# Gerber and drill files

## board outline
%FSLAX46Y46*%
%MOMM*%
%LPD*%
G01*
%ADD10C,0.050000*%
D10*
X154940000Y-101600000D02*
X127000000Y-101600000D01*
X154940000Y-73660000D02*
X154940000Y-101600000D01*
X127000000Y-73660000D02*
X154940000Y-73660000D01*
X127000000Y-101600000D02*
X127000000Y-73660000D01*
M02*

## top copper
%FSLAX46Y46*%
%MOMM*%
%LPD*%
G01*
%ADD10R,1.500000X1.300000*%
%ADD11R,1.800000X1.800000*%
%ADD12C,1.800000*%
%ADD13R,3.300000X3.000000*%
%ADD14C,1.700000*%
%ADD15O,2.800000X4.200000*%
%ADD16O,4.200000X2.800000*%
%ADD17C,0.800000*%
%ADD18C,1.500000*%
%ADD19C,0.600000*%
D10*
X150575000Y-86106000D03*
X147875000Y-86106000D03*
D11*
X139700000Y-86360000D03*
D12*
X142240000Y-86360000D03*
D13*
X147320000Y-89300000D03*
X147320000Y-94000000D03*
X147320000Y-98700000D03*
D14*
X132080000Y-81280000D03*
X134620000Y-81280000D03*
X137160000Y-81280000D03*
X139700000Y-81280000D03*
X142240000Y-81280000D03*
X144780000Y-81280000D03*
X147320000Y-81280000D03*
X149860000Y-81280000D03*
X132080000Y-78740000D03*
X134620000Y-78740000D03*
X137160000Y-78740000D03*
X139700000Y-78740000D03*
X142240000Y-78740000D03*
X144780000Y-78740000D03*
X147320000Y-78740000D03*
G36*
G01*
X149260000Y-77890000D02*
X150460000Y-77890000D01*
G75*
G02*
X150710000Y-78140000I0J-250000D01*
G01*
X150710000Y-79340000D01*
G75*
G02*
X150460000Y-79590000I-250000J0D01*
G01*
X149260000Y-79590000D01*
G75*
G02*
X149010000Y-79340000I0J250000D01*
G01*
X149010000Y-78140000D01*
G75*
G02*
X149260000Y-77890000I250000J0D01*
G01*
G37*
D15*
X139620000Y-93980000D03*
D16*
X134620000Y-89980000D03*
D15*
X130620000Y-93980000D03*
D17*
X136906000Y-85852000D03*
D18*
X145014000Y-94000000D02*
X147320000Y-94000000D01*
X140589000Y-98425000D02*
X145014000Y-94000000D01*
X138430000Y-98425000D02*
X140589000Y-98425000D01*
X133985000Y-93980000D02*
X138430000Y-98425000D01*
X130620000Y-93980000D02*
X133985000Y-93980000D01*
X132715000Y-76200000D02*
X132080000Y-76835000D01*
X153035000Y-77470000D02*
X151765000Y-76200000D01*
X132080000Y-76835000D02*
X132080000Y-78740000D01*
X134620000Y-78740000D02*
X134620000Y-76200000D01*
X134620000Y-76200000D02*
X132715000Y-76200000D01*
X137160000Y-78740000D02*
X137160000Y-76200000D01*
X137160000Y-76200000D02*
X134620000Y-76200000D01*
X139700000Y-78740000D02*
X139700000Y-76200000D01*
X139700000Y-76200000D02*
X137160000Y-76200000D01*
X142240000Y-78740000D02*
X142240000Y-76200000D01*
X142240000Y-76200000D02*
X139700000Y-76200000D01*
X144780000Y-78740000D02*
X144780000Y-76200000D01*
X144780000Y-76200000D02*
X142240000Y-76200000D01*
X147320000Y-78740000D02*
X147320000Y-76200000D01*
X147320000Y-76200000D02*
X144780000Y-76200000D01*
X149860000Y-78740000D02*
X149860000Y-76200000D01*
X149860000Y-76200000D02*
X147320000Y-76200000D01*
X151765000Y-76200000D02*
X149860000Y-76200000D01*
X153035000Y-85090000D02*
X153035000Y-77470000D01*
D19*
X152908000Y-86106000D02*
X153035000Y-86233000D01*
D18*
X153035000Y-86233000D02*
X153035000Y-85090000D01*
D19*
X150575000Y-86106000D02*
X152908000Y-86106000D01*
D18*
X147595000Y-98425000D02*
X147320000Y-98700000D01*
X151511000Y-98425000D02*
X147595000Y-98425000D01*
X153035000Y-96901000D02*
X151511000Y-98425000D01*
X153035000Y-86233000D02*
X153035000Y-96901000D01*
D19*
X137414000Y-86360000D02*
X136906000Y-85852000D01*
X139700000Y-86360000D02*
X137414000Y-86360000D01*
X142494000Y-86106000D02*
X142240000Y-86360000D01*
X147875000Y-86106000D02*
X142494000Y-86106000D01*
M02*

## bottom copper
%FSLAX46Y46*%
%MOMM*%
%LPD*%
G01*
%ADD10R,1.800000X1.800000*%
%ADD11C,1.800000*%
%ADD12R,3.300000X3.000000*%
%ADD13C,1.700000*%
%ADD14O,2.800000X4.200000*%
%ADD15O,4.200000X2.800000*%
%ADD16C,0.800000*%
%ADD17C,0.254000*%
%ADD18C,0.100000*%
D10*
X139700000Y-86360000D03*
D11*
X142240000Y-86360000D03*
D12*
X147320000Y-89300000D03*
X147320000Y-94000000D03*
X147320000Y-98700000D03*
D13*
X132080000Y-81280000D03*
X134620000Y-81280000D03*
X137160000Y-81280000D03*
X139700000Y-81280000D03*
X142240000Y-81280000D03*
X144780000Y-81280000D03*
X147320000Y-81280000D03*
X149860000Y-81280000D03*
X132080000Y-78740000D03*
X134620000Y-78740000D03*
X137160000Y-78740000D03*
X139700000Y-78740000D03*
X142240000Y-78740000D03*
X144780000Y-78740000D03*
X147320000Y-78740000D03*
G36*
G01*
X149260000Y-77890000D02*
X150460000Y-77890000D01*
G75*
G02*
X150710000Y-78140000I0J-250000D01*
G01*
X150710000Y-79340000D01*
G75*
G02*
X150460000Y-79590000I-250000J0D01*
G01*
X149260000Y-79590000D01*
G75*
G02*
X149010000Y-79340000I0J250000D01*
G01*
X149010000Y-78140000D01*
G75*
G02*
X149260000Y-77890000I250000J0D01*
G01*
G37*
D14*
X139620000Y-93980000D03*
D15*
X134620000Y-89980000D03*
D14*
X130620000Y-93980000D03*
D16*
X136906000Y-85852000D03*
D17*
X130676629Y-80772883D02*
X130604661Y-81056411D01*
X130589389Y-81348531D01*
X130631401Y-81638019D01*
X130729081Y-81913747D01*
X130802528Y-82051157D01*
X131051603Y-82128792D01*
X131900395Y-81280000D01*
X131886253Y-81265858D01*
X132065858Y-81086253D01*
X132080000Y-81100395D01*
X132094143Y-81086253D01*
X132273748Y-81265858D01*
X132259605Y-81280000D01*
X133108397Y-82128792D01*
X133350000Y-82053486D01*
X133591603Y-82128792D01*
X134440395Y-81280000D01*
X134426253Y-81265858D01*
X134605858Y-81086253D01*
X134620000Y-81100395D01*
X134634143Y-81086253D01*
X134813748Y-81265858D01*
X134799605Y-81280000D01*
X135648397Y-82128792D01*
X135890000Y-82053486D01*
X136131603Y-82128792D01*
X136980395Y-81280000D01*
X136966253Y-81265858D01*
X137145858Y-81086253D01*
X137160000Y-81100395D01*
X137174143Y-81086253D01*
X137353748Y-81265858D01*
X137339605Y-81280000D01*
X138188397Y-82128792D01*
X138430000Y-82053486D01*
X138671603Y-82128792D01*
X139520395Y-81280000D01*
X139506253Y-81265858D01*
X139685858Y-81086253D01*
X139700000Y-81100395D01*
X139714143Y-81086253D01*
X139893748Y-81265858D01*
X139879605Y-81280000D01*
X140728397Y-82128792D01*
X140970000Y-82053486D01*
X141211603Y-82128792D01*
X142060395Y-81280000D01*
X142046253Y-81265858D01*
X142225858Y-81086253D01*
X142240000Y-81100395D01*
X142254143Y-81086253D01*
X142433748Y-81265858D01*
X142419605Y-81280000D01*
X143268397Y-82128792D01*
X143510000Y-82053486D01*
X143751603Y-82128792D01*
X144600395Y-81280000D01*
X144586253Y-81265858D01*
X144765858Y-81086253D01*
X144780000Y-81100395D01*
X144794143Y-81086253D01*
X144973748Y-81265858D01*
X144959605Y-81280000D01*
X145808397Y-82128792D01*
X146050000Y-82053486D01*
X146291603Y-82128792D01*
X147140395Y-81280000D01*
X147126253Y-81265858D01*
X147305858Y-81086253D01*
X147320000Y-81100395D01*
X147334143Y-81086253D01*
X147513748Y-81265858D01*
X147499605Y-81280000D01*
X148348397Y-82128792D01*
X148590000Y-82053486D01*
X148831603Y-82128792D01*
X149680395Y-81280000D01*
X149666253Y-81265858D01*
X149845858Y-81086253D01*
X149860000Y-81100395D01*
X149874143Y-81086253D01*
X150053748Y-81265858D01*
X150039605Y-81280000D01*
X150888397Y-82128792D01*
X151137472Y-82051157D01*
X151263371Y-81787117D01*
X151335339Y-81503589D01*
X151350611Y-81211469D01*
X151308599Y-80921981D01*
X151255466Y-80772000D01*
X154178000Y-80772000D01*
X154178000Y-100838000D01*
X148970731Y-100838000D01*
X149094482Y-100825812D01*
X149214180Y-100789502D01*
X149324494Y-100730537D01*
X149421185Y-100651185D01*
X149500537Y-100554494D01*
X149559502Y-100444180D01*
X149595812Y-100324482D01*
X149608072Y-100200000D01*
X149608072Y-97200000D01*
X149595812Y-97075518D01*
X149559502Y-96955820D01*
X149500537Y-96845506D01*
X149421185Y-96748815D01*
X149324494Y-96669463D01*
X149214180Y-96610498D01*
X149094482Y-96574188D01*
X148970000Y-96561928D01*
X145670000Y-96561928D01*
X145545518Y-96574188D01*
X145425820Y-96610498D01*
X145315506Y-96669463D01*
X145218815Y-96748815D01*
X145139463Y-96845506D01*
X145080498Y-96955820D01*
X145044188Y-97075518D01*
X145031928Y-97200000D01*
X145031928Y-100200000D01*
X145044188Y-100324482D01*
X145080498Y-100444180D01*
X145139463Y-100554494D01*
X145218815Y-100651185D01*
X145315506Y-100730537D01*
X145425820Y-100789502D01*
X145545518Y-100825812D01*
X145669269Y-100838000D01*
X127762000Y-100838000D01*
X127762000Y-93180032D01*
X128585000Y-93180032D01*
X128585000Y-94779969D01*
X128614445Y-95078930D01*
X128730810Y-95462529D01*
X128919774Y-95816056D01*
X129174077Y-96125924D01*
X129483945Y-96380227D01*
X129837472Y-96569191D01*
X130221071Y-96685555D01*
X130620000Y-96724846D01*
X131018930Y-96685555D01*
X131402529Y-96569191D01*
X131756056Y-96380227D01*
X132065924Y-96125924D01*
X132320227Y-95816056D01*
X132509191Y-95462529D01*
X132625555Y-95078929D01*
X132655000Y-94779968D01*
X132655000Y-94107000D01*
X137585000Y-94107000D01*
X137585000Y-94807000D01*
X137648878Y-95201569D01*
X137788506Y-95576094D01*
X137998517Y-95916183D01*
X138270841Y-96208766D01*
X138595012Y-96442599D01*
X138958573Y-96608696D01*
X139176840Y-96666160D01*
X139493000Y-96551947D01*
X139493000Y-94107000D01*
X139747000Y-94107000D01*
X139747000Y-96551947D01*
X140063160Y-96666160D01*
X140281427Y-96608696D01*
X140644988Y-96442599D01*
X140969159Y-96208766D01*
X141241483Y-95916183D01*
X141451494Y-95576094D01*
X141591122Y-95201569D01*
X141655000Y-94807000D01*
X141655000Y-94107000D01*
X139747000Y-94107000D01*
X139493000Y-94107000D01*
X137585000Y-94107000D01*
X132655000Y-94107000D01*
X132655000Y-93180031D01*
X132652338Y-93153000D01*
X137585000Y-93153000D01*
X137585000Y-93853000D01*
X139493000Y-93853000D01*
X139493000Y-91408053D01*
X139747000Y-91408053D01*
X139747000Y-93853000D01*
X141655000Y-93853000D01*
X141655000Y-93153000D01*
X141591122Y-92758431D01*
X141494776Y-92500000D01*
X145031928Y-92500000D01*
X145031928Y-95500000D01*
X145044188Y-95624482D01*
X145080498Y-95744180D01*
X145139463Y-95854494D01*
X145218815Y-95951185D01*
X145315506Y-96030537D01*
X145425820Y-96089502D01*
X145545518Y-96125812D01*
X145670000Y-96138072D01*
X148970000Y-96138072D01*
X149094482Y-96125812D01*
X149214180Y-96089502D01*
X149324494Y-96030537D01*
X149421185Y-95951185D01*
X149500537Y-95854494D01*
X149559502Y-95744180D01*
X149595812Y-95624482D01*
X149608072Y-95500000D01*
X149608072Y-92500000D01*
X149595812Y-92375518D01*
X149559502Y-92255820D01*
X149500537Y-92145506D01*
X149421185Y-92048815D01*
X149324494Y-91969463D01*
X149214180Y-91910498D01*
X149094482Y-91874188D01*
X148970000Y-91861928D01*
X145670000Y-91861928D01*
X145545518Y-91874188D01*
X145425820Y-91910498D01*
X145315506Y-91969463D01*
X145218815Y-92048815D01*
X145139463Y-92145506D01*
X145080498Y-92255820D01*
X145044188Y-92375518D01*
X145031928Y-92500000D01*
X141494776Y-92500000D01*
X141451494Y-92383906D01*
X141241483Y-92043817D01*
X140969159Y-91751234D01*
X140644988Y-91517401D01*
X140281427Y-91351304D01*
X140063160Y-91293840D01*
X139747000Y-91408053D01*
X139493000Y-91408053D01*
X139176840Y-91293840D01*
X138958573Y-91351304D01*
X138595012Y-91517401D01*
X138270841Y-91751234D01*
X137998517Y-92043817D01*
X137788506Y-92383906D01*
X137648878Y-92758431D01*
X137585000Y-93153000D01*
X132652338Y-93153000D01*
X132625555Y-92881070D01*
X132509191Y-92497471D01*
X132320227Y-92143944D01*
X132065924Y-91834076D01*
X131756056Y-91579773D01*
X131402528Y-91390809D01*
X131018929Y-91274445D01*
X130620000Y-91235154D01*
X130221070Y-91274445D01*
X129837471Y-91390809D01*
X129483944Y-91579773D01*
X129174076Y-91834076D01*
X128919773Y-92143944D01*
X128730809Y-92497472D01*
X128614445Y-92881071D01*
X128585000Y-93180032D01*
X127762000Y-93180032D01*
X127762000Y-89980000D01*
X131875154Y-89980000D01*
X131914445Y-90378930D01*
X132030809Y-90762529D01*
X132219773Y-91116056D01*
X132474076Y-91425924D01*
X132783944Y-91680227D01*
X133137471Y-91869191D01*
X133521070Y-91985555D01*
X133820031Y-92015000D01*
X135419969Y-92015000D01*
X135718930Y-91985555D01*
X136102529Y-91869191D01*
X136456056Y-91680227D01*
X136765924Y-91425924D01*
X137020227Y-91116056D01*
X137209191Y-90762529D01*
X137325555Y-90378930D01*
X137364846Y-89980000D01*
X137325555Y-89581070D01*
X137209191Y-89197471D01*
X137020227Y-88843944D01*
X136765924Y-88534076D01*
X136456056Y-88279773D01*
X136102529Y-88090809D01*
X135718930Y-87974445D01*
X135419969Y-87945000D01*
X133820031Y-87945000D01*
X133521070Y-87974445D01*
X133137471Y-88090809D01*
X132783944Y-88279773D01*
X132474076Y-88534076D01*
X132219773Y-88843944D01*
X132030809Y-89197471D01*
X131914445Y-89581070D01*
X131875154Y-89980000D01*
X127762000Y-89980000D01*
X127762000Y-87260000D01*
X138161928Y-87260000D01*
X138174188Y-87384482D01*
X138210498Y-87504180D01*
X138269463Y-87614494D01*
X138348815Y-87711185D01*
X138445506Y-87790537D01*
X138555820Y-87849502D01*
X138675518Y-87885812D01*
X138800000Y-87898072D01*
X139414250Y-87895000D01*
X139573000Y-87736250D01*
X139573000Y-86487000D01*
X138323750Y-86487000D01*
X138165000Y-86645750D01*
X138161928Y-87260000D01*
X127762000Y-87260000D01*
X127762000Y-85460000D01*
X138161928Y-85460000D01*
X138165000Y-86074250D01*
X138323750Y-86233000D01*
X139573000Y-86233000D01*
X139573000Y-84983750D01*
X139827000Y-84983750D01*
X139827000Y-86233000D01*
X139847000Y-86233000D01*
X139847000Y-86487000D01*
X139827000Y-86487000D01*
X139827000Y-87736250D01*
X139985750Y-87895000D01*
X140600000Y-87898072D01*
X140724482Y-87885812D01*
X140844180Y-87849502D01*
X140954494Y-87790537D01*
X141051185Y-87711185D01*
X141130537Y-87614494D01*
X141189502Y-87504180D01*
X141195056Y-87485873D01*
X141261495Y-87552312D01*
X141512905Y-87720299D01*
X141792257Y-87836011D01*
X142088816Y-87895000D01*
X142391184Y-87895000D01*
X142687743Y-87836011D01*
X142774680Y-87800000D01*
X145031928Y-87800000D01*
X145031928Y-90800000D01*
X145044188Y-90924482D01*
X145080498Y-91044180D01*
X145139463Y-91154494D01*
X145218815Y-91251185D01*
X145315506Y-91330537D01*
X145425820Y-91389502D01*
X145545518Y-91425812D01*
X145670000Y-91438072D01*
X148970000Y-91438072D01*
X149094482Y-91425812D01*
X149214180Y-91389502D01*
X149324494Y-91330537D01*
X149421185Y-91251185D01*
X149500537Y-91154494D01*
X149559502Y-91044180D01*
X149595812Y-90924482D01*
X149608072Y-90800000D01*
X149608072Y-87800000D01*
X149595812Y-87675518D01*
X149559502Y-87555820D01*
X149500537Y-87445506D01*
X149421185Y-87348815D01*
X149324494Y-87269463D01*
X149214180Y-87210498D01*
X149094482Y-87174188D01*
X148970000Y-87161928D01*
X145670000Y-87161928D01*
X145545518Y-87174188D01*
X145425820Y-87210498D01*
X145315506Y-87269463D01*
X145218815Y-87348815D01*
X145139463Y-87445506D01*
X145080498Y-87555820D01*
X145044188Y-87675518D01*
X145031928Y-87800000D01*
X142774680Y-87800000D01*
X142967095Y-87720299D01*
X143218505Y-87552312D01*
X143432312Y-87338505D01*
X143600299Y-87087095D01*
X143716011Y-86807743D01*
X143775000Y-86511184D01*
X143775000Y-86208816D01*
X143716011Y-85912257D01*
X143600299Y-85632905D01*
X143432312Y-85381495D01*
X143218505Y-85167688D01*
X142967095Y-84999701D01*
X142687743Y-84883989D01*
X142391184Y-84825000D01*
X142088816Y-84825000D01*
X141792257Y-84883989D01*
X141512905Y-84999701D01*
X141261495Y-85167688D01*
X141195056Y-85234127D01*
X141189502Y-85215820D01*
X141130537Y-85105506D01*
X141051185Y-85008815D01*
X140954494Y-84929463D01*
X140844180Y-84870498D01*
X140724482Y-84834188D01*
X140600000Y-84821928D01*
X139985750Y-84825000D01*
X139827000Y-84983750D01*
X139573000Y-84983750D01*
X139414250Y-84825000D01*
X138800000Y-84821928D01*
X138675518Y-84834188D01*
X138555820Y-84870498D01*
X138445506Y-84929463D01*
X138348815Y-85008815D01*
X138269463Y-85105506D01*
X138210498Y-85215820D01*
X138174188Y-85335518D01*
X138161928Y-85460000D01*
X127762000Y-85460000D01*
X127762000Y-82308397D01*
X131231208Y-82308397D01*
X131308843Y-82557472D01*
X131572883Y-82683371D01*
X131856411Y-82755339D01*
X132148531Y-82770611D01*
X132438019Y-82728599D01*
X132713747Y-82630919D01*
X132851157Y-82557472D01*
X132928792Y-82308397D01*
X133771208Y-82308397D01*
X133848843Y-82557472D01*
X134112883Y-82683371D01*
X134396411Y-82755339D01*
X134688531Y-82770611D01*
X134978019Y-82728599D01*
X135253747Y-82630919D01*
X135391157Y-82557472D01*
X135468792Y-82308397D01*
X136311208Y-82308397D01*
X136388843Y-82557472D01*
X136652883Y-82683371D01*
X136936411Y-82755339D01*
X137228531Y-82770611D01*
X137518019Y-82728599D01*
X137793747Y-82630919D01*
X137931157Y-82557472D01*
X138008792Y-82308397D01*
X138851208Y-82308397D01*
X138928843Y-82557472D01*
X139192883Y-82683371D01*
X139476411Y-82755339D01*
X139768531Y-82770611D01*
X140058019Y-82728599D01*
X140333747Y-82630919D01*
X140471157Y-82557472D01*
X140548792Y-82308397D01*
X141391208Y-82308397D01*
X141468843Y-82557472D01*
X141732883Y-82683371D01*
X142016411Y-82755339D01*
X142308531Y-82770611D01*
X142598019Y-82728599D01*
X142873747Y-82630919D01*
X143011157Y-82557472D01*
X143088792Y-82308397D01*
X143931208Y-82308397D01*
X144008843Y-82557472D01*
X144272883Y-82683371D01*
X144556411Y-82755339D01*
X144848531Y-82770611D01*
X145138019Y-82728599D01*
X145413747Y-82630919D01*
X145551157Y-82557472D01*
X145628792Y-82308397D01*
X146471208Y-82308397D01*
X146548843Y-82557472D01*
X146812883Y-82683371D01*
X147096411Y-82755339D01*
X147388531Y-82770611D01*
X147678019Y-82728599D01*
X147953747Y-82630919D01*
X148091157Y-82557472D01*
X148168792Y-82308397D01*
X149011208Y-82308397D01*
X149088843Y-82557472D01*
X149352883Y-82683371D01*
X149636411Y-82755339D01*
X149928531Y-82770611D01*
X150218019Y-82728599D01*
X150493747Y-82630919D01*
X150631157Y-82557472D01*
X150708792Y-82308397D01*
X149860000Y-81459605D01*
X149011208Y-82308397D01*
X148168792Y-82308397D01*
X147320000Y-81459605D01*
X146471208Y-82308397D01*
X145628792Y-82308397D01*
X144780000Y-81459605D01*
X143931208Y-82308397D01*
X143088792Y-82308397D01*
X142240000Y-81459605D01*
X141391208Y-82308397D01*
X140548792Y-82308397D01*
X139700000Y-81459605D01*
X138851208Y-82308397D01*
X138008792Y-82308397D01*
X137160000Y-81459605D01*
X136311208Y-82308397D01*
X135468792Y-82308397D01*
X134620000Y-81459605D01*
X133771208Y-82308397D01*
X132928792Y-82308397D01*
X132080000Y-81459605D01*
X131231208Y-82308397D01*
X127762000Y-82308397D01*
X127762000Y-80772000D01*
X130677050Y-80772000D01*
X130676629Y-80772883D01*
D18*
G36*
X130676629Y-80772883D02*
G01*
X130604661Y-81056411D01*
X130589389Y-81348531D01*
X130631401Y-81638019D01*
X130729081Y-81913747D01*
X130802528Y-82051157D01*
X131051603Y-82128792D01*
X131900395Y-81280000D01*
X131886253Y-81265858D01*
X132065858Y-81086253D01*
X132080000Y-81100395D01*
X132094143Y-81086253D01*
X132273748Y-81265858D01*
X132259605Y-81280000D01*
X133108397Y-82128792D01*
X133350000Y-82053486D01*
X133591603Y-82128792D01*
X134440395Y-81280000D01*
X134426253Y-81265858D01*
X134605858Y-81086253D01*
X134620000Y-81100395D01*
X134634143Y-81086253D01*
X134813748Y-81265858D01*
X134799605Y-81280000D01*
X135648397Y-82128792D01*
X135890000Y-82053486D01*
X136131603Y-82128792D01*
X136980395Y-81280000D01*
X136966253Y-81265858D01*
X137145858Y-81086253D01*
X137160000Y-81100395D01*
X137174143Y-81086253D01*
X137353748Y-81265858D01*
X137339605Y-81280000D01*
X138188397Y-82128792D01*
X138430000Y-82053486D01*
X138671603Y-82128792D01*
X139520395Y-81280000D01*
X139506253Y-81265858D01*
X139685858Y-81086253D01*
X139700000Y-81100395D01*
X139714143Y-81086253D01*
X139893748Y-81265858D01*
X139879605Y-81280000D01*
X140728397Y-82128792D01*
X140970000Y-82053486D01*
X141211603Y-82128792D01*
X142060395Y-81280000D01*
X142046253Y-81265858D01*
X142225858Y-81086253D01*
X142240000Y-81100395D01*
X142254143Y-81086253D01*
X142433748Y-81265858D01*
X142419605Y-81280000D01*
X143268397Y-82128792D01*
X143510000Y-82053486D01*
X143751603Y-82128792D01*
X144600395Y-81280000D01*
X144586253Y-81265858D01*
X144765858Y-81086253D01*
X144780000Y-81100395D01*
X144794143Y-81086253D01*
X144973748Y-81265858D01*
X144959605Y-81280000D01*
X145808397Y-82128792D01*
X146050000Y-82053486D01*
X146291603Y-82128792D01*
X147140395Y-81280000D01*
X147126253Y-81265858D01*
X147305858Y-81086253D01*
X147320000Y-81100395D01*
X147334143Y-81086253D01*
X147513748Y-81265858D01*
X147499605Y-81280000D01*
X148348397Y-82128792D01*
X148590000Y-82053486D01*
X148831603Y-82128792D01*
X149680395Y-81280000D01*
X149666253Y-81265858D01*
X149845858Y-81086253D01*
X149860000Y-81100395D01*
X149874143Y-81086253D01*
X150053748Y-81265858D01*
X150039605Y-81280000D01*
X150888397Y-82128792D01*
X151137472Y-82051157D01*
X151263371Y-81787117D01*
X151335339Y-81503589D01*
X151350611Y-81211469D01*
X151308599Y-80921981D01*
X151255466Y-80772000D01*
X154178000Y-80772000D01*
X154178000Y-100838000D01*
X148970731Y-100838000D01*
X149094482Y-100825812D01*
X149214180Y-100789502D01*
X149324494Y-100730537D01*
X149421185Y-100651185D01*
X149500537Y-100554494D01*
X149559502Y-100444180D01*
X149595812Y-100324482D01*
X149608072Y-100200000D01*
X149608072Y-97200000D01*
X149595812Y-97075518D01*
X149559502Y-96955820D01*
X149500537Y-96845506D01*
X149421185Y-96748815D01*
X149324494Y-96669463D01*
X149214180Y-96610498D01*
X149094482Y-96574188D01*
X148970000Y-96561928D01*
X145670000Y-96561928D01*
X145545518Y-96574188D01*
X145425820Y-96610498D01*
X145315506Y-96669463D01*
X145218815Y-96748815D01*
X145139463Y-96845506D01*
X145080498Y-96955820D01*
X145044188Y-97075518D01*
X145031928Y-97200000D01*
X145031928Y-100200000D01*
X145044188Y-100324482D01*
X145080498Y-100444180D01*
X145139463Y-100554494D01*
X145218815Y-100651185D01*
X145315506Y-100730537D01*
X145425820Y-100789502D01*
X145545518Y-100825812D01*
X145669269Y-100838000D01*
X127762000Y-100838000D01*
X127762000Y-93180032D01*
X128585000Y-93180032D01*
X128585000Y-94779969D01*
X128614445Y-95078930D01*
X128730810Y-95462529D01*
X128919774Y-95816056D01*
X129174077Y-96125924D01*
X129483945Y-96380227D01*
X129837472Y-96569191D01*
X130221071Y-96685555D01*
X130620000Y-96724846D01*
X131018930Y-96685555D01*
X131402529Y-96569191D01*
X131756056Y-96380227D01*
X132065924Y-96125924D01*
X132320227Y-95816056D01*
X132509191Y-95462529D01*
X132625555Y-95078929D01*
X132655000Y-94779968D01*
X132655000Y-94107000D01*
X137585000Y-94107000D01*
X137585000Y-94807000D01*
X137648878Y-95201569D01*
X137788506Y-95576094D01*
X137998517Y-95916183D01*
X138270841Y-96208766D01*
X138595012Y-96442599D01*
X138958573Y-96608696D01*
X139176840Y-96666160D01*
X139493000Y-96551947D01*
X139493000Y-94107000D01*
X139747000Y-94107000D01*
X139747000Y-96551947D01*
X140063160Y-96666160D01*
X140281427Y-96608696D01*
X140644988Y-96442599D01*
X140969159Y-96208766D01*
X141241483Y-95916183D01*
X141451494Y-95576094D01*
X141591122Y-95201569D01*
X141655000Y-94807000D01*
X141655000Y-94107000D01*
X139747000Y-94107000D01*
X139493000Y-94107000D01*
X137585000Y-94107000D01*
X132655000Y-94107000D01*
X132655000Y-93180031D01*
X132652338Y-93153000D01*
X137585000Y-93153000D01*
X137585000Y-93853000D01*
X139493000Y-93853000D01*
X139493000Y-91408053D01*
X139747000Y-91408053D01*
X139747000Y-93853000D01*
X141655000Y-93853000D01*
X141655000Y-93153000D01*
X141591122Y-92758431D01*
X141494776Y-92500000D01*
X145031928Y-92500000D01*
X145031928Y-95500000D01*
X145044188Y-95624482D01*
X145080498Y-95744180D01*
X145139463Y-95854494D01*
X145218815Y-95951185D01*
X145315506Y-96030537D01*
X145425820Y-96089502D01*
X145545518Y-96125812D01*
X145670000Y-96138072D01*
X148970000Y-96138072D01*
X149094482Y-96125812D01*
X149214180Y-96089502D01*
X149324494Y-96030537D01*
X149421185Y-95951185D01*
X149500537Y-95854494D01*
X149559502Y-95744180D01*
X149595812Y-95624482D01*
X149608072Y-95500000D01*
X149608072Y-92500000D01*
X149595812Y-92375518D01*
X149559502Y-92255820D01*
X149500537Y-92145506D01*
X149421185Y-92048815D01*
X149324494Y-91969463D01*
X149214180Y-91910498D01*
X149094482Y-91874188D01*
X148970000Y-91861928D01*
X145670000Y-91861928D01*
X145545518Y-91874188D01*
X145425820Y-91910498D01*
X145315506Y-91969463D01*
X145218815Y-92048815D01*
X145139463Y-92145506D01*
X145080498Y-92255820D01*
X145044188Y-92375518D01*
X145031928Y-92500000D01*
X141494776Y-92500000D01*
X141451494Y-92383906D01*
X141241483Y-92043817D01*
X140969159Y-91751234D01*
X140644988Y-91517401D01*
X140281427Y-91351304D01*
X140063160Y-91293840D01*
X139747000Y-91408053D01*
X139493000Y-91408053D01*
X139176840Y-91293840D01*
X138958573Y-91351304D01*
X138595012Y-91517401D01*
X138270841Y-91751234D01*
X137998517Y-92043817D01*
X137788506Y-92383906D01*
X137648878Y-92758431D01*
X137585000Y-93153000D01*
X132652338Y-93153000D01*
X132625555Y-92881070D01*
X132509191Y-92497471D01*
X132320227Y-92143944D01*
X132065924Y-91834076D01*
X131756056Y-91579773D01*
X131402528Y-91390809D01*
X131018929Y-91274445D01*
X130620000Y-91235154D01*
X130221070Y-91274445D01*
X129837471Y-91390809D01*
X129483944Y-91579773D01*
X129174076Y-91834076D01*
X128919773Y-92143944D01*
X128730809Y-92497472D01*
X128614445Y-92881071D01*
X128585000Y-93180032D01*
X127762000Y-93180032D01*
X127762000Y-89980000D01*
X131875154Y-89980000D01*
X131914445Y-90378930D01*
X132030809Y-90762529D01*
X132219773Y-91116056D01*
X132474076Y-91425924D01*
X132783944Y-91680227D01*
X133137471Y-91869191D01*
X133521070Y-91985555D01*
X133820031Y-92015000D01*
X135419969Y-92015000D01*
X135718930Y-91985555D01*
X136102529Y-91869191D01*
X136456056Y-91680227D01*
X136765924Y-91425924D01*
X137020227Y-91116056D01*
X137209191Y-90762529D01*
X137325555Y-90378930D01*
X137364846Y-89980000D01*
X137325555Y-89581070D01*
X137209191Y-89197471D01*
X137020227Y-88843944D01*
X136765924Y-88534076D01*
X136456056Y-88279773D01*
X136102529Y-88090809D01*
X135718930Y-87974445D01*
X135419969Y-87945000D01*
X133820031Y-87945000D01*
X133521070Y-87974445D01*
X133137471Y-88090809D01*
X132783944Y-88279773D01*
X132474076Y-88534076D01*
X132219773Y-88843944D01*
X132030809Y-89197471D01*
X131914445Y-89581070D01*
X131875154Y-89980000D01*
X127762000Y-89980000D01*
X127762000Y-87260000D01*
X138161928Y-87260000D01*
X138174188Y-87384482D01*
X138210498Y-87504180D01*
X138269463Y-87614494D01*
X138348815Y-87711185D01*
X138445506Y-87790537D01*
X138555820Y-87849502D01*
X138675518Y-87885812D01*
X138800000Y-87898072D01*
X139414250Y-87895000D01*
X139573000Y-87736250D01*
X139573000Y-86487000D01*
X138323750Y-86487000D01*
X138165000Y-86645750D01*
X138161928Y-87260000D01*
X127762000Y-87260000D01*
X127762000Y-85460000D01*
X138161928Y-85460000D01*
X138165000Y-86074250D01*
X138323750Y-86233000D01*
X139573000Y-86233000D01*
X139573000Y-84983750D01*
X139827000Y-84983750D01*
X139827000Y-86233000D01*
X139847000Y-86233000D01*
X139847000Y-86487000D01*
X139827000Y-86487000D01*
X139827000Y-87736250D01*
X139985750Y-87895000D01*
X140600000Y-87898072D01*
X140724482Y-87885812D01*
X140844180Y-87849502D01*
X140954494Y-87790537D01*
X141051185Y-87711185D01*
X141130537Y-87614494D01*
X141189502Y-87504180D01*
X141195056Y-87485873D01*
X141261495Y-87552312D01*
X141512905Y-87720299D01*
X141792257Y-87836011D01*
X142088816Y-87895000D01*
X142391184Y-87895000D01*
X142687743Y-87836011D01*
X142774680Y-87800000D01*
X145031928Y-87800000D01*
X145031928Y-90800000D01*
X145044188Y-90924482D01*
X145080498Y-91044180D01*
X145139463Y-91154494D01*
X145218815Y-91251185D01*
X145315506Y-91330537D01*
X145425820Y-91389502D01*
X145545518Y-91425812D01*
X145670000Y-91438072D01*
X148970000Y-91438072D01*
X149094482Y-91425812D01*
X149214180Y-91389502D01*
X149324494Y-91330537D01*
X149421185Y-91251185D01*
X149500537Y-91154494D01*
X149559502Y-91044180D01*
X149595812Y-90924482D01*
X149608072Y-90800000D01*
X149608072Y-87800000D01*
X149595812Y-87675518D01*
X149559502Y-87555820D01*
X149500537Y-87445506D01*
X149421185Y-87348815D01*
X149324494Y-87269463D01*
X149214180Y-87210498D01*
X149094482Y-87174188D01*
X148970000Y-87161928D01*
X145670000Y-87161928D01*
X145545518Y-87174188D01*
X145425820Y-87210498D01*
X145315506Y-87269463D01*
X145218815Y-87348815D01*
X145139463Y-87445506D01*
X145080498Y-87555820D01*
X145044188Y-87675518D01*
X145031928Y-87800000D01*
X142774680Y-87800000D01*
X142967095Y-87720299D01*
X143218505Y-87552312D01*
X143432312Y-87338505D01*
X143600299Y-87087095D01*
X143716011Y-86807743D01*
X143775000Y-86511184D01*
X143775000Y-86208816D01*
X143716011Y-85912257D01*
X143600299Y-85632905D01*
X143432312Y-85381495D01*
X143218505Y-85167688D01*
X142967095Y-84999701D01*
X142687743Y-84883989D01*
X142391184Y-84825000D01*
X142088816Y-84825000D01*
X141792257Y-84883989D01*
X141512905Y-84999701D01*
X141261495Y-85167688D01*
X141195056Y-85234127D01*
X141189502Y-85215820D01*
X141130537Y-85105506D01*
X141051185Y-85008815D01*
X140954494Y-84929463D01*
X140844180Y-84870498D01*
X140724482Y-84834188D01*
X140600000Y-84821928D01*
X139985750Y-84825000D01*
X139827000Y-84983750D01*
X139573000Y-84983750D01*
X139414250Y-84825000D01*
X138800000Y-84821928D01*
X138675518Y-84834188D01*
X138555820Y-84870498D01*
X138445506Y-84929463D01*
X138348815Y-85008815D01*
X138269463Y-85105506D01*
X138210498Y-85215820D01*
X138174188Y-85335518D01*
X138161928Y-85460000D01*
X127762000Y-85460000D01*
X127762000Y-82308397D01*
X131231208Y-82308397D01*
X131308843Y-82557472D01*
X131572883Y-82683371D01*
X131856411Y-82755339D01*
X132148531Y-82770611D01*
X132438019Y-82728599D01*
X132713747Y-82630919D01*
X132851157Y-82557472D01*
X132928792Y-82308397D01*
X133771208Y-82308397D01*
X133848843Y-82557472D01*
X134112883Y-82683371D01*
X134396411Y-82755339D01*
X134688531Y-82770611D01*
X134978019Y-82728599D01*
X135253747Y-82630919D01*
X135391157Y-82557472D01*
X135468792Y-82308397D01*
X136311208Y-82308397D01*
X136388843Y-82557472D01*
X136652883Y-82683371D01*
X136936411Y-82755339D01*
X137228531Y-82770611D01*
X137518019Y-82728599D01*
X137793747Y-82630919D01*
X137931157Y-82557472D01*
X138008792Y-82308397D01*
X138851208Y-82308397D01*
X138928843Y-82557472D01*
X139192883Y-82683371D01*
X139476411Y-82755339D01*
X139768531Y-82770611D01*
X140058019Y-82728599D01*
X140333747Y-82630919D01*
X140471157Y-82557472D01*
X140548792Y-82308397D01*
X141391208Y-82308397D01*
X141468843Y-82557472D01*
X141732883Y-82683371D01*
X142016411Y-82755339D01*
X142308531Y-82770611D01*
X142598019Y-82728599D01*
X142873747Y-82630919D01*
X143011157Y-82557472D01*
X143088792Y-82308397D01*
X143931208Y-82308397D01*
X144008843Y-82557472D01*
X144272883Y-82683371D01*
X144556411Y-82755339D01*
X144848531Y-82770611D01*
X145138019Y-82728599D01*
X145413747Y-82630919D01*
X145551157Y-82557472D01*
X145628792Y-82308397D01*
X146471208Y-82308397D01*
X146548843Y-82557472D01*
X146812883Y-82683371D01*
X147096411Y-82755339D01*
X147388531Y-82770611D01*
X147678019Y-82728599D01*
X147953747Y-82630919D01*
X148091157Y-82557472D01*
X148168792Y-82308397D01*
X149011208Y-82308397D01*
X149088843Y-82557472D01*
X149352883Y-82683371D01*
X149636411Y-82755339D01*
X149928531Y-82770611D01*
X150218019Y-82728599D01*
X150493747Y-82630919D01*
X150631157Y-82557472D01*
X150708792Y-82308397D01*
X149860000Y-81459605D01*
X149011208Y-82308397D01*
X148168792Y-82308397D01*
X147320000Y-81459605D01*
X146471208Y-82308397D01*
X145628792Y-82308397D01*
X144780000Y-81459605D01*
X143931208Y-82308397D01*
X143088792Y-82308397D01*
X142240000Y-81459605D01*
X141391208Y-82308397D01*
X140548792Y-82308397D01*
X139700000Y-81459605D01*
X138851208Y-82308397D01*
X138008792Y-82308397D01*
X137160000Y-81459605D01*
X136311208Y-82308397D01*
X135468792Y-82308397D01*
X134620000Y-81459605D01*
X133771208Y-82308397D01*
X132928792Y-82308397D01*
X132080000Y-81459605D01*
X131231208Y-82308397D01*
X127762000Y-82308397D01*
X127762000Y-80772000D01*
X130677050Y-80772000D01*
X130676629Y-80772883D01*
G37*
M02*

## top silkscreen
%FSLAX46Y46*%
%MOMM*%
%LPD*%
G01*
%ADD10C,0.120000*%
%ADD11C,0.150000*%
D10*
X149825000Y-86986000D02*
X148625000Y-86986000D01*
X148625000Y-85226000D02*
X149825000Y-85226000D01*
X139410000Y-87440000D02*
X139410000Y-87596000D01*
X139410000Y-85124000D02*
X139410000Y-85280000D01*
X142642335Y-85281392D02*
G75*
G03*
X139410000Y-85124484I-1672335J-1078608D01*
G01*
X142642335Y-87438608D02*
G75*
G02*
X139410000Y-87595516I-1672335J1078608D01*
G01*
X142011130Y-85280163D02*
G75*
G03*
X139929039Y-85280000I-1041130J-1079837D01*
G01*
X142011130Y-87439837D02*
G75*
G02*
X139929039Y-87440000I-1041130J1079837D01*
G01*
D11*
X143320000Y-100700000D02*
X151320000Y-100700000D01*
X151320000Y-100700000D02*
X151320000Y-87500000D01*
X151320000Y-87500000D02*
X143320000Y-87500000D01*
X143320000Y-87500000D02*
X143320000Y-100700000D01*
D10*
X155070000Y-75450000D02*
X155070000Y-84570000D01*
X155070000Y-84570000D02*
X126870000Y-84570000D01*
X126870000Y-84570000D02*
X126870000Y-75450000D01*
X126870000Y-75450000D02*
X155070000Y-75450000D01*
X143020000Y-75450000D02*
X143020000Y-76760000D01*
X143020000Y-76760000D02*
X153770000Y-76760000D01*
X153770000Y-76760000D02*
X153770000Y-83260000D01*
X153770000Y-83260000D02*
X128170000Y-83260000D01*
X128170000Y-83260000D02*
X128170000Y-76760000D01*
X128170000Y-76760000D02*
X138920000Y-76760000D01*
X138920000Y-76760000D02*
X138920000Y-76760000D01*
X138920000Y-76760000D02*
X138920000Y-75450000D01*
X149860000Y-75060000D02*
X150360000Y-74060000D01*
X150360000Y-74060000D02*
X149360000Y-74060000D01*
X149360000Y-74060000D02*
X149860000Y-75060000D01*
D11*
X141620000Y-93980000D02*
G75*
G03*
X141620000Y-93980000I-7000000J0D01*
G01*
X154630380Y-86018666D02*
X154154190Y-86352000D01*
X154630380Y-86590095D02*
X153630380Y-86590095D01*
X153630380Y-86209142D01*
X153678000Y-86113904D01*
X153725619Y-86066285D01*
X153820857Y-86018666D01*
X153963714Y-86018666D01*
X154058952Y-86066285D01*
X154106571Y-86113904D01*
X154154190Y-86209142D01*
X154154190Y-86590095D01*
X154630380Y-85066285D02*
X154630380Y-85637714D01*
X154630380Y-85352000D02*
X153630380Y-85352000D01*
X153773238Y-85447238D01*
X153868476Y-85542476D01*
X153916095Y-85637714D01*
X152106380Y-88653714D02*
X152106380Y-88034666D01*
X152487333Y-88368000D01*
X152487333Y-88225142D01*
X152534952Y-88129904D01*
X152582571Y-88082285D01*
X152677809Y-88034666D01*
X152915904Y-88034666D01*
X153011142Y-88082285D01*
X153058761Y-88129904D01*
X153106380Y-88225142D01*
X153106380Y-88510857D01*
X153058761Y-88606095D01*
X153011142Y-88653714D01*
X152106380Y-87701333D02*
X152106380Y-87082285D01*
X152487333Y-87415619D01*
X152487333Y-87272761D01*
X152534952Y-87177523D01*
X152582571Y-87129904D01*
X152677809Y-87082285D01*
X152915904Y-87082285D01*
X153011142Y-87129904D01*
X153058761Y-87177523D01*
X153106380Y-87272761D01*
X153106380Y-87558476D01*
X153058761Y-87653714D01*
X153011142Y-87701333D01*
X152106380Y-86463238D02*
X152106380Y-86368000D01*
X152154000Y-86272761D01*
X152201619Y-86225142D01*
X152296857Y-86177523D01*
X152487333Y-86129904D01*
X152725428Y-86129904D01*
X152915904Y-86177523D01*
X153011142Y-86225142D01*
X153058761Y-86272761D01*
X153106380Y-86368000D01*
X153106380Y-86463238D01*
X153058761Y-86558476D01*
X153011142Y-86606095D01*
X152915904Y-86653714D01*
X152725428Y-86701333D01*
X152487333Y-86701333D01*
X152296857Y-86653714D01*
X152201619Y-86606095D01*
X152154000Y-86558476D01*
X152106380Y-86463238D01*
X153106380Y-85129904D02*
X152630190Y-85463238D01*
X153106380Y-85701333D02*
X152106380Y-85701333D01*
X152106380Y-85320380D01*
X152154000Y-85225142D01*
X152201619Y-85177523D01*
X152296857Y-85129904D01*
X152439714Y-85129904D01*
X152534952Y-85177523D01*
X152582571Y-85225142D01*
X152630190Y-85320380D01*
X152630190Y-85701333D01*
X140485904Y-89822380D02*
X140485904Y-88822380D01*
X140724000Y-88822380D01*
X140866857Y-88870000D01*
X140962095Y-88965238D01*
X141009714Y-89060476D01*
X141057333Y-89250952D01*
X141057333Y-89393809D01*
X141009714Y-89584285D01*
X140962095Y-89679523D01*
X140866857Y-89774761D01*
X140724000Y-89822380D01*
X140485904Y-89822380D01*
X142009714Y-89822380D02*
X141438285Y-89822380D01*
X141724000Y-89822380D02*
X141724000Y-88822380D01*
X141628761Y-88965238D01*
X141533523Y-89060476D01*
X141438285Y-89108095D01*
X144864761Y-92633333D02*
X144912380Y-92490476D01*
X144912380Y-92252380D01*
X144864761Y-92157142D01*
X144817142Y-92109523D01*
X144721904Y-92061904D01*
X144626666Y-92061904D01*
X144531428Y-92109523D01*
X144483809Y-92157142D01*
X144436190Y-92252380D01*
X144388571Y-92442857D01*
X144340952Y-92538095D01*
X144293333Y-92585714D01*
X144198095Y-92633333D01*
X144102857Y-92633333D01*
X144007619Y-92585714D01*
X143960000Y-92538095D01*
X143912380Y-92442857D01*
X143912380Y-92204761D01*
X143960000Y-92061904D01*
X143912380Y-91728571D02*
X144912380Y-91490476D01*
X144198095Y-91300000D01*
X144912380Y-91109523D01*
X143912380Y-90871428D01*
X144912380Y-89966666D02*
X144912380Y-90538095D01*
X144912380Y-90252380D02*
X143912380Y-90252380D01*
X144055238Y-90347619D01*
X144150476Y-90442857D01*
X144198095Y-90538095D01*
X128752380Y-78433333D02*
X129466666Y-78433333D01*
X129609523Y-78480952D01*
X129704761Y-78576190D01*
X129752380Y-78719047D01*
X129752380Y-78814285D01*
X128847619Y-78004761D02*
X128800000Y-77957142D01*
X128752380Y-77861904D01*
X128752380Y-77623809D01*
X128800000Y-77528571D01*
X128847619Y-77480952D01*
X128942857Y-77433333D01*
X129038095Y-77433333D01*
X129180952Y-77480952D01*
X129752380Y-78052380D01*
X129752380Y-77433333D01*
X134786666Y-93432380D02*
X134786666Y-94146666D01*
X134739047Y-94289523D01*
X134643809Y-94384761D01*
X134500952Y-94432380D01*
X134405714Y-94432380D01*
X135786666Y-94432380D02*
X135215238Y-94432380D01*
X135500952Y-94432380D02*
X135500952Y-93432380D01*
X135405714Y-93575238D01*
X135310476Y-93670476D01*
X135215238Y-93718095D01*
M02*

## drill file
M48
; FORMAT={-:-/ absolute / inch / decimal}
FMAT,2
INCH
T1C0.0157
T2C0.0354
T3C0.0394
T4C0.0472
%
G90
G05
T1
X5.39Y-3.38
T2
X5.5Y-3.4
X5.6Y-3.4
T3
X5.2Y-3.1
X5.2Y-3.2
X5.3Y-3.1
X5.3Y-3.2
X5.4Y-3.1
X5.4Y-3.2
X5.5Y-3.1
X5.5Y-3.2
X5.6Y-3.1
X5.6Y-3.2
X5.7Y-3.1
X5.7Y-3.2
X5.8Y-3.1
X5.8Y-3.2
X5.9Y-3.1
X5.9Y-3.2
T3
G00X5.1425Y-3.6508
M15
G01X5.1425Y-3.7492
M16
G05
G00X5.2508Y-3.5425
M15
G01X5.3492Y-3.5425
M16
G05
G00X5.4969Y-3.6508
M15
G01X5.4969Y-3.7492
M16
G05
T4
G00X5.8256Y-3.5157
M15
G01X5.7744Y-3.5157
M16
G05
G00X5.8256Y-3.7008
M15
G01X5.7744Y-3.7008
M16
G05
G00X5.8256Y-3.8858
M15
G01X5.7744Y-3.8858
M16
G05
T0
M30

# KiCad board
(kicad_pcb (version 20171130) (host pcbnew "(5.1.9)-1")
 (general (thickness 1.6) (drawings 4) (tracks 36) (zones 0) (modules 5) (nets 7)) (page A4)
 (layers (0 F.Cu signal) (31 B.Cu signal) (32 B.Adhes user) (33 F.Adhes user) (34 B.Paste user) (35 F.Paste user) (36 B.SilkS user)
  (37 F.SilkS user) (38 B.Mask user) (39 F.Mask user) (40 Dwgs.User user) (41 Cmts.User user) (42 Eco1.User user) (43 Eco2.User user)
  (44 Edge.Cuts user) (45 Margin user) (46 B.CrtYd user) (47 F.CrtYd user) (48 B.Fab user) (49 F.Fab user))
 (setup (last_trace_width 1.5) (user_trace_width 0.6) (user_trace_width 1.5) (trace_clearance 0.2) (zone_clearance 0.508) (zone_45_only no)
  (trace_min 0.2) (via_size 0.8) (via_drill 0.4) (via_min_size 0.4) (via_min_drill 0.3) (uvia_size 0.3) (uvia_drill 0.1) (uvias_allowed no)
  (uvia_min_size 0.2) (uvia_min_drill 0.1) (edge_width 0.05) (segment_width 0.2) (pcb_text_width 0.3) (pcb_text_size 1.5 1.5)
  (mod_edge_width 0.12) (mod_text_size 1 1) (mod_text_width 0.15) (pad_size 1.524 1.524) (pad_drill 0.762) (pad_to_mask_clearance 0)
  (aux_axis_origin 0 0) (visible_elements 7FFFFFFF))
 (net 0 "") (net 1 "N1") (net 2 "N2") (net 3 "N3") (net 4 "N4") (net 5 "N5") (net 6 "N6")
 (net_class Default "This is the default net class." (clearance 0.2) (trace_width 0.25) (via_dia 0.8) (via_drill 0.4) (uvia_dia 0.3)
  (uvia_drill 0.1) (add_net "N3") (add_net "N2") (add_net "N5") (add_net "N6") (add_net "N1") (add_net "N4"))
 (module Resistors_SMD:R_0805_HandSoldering (layer F.Cu) (at 149.225 86.106 180)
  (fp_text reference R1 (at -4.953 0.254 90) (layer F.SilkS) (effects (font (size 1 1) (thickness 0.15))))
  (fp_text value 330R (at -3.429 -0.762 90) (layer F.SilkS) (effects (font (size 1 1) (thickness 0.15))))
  (fp_line (start -0.6 -0.88) (end 0.6 -0.88) (layer F.SilkS) (width 0.12))
  (fp_line (start 0.6 0.88) (end -0.6 0.88) (layer F.SilkS) (width 0.12))
  (pad 1 smd rect (at -1.35 0 180) (size 1.5 1.3) (layers F.Cu F.Paste F.Mask) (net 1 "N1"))
  (pad 2 smd rect (at 1.35 0 180) (size 1.5 1.3) (layers F.Cu F.Paste F.Mask) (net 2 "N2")))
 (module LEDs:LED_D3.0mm (layer F.Cu) (at 139.7 86.36)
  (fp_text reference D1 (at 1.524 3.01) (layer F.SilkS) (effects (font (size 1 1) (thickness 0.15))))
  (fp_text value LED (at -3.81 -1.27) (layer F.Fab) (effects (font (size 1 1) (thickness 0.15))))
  (fp_line (start -0.29 1.08) (end -0.29 1.236) (layer F.SilkS) (width 0.12))
  (fp_line (start -0.29 -1.236) (end -0.29 -1.08) (layer F.SilkS) (width 0.12))
  (fp_arc (start 1.27 0) (end -0.29 -1.235516) (angle 108.8) (layer F.SilkS) (width 0.12))
  (fp_arc (start 1.27 0) (end -0.29 1.235516) (angle -108.8) (layer F.SilkS) (width 0.12))
  (fp_arc (start 1.27 0) (end 0.229039 -1.08) (angle 87.9) (layer F.SilkS) (width 0.12))
  (fp_arc (start 1.27 0) (end 0.229039 1.08) (angle -87.9) (layer F.SilkS) (width 0.12))
  (pad 1 thru_hole rect (at 0 0) (size 1.8 1.8) (drill 0.9) (layers *.Cu *.Mask) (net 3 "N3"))
  (pad 2 thru_hole circle (at 2.54 0) (size 1.8 1.8) (drill 0.9) (layers *.Cu *.Mask) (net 2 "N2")))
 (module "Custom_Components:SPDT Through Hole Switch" (layer F.Cu) (at 147.32 98.7 180)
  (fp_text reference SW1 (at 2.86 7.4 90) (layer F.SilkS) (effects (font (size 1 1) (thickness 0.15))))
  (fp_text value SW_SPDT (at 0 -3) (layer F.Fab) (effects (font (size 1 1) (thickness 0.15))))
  (fp_line (start 4 -2) (end -4 -2) (layer F.SilkS) (width 0.15))
  (fp_line (start -4 -2) (end -4 11.2) (layer F.SilkS) (width 0.15))
  (fp_line (start -4 11.2) (end 4 11.2) (layer F.SilkS) (width 0.15))
  (fp_line (start 4 11.2) (end 4 -2) (layer F.SilkS) (width 0.15))
  (pad 3 thru_hole rect (at 0 9.4 180) (size 3.3 3) (drill oval 2.5 1.2) (layers *.Cu *.Mask) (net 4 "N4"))
  (pad 2 thru_hole rect (at 0 4.7 180) (size 3.3 3) (drill oval 2.5 1.2) (layers *.Cu *.Mask) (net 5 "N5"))
  (pad 1 thru_hole rect (at 0 0 180) (size 3.3 3) (drill oval 2.5 1.2) (layers *.Cu *.Mask) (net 1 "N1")))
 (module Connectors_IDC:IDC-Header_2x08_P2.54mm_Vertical (layer F.Cu) (at 149.86 78.74 270)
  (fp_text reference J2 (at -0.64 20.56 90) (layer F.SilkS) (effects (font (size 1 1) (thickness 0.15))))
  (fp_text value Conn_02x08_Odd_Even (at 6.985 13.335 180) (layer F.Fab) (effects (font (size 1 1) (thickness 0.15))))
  (fp_line (start -3.29 -5.21) (end 5.83 -5.21) (layer F.SilkS) (width 0.12))
  (fp_line (start 5.83 -5.21) (end 5.83 22.99) (layer F.SilkS) (width 0.12))
  (fp_line (start 5.83 22.99) (end -3.29 22.99) (layer F.SilkS) (width 0.12))
  (fp_line (start -3.29 22.99) (end -3.29 -5.21) (layer F.SilkS) (width 0.12))
  (fp_line (start -3.29 6.84) (end -1.98 6.84) (layer F.SilkS) (width 0.12))
  (fp_line (start -1.98 6.84) (end -1.98 -3.91) (layer F.SilkS) (width 0.12))
  (fp_line (start -1.98 -3.91) (end 4.52 -3.91) (layer F.SilkS) (width 0.12))
  (fp_line (start 4.52 -3.91) (end 4.52 21.69) (layer F.SilkS) (width 0.12))
  (fp_line (start 4.52 21.69) (end -1.98 21.69) (layer F.SilkS) (width 0.12))
  (fp_line (start -1.98 21.69) (end -1.98 10.94) (layer F.SilkS) (width 0.12))
  (fp_line (start -1.98 10.94) (end -1.98 10.94) (layer F.SilkS) (width 0.12))
  (fp_line (start -1.98 10.94) (end -3.29 10.94) (layer F.SilkS) (width 0.12))
  (fp_line (start -3.68 0) (end -4.68 -0.5) (layer F.SilkS) (width 0.12))
  (fp_line (start -4.68 -0.5) (end -4.68 0.5) (layer F.SilkS) (width 0.12))
  (fp_line (start -4.68 0.5) (end -3.68 0) (layer F.SilkS) (width 0.12))
  (pad 16 thru_hole circle (at 2.54 17.78 270) (size 1.7 1.7) (drill 1) (layers *.Cu *.Mask) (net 3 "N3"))
  (pad 14 thru_hole circle (at 2.54 15.24 270) (size 1.7 1.7) (drill 1) (layers *.Cu *.Mask) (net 3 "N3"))
  (pad 12 thru_hole circle (at 2.54 12.7 270) (size 1.7 1.7) (drill 1) (layers *.Cu *.Mask) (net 3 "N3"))
  (pad 10 thru_hole circle (at 2.54 10.16 270) (size 1.7 1.7) (drill 1) (layers *.Cu *.Mask) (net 3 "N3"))
  (pad 8 thru_hole circle (at 2.54 7.62 270) (size 1.7 1.7) (drill 1) (layers *.Cu *.Mask) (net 3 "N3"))
  (pad 6 thru_hole circle (at 2.54 5.08 270) (size 1.7 1.7) (drill 1) (layers *.Cu *.Mask) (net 3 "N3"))
  (pad 4 thru_hole circle (at 2.54 2.54 270) (size 1.7 1.7) (drill 1) (layers *.Cu *.Mask) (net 3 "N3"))
  (pad 2 thru_hole circle (at 2.54 0 270) (size 1.7 1.7) (drill 1) (layers *.Cu *.Mask) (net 3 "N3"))
  (pad 15 thru_hole circle (at 0 17.78 270) (size 1.7 1.7) (drill 1) (layers *.Cu *.Mask) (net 1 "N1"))
  (pad 13 thru_hole circle (at 0 15.24 270) (size 1.7 1.7) (drill 1) (layers *.Cu *.Mask) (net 1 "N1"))
  (pad 11 thru_hole circle (at 0 12.7 270) (size 1.7 1.7) (drill 1) (layers *.Cu *.Mask) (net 1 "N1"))
  (pad 9 thru_hole circle (at 0 10.16 270) (size 1.7 1.7) (drill 1) (layers *.Cu *.Mask) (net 1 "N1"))
  (pad 7 thru_hole circle (at 0 7.62 270) (size 1.7 1.7) (drill 1) (layers *.Cu *.Mask) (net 1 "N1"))
  (pad 5 thru_hole circle (at 0 5.08 270) (size 1.7 1.7) (drill 1) (layers *.Cu *.Mask) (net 1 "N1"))
  (pad 3 thru_hole circle (at 0 2.54 270) (size 1.7 1.7) (drill 1) (layers *.Cu *.Mask) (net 1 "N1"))
  (pad 1 thru_hole roundrect (at 0 0 270) (size 1.7 1.7) (drill 1) (layers *.Cu *.Mask) (roundrect_rratio 0.1470588235294118) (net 1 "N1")))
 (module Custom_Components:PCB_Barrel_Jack (layer F.Cu) (at 134.62 93.98)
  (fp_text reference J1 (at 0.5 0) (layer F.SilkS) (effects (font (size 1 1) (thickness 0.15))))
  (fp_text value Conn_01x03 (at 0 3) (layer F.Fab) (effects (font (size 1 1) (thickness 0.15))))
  (fp_circle (center 0 0) (end 7 0) (layer F.SilkS) (width 0.15))
  (pad 3 thru_hole oval (at 5 0) (size 2.8 4.2) (drill oval 1 3.5) (layers *.Cu *.Mask) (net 3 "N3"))
  (pad 2 thru_hole oval (at 0 -4) (size 4.2 2.8) (drill oval 3.5 1) (layers *.Cu *.Mask) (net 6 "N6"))
  (pad 1 thru_hole oval (at -4 0) (size 2.8 4.2) (drill oval 1 3.5) (layers *.Cu *.Mask) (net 5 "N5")))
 (gr_line (start 154.94 101.6) (end 127 101.6) (layer Edge.Cuts) (width 0.05))
 (gr_line (start 154.94 73.66) (end 154.94 101.6) (layer Edge.Cuts) (width 0.05))
 (gr_line (start 127 73.66) (end 154.94 73.66) (layer Edge.Cuts) (width 0.05))
 (gr_line (start 127 101.6) (end 127 73.66) (layer Edge.Cuts) (width 0.05))
 (segment (start 145.014 94) (end 147.32 94) (width 1.5) (layer F.Cu) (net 5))
 (segment (start 140.589 98.425) (end 145.014 94) (width 1.5) (layer F.Cu) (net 5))
 (segment (start 138.43 98.425) (end 140.589 98.425) (width 1.5) (layer F.Cu) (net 5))
 (segment (start 133.985 93.98) (end 138.43 98.425) (width 1.5) (layer F.Cu) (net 5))
 (segment (start 130.62 93.98) (end 133.985 93.98) (width 1.5) (layer F.Cu) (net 5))
 (segment (start 132.715 76.2) (end 132.08 76.835) (width 1.5) (layer F.Cu) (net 1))
 (segment (start 153.035 77.47) (end 151.765 76.2) (width 1.5) (layer F.Cu) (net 1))
 (segment (start 132.08 76.835) (end 132.08 78.74) (width 1.5) (layer F.Cu) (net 1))
 (segment (start 134.62 78.74) (end 134.62 76.2) (width 1.5) (layer F.Cu) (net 1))
 (segment (start 134.62 76.2) (end 132.715 76.2) (width 1.5) (layer F.Cu) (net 1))
 (segment (start 137.16 78.74) (end 137.16 76.2) (width 1.5) (layer F.Cu) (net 1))
 (segment (start 137.16 76.2) (end 134.62 76.2) (width 1.5) (layer F.Cu) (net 1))
 (segment (start 139.7 78.74) (end 139.7 76.2) (width 1.5) (layer F.Cu) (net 1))
 (segment (start 139.7 76.2) (end 137.16 76.2) (width 1.5) (layer F.Cu) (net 1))
 (segment (start 142.24 78.74) (end 142.24 76.2) (width 1.5) (layer F.Cu) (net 1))
 (segment (start 142.24 76.2) (end 139.7 76.2) (width 1.5) (layer F.Cu) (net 1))
 (segment (start 144.78 78.74) (end 144.78 76.2) (width 1.5) (layer F.Cu) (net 1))
 (segment (start 144.78 76.2) (end 142.24 76.2) (width 1.5) (layer F.Cu) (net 1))
 (segment (start 147.32 78.74) (end 147.32 76.2) (width 1.5) (layer F.Cu) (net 1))
 (segment (start 147.32 76.2) (end 144.78 76.2) (width 1.5) (layer F.Cu) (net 1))
 (segment (start 149.86 78.74) (end 149.86 76.2) (width 1.5) (layer F.Cu) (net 1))
 (segment (start 149.86 76.2) (end 147.32 76.2) (width 1.5) (layer F.Cu) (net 1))
 (segment (start 151.765 76.2) (end 149.86 76.2) (width 1.5) (layer F.Cu) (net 1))
 (segment (start 153.035 85.09) (end 153.035 77.47) (width 1.5) (layer F.Cu) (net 1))
 (segment (start 152.908 86.106) (end 153.035 86.233) (width 0.6) (layer F.Cu) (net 1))
 (segment (start 153.035 86.233) (end 153.035 85.09) (width 1.5) (layer F.Cu) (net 1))
 (segment (start 150.575 86.106) (end 152.908 86.106) (width 0.6) (layer F.Cu) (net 1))
 (segment (start 147.595 98.425) (end 147.32 98.7) (width 1.5) (layer F.Cu) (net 1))
 (segment (start 151.511 98.425) (end 147.595 98.425) (width 1.5) (layer F.Cu) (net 1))
 (segment (start 153.035 96.901) (end 151.511 98.425) (width 1.5) (layer F.Cu) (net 1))
 (segment (start 153.035 86.233) (end 153.035 96.901) (width 1.5) (layer F.Cu) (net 1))
 (via (at 136.906 85.852) (size 0.8) (drill 0.4) (layers F.Cu B.Cu) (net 3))
 (segment (start 137.414 86.36) (end 136.906 85.852) (width 0.6) (layer F.Cu) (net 3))
 (segment (start 139.7 86.36) (end 137.414 86.36) (width 0.6) (layer F.Cu) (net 3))
 (segment (start 142.494 86.106) (end 142.24 86.36) (width 0.6) (layer F.Cu) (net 2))
 (segment (start 147.875 86.106) (end 142.494 86.106) (width 0.6) (layer F.Cu) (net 2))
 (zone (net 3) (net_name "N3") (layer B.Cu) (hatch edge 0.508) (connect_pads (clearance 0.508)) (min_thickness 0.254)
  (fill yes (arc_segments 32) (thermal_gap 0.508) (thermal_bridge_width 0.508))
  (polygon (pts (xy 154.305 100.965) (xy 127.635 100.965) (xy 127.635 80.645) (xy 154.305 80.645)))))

